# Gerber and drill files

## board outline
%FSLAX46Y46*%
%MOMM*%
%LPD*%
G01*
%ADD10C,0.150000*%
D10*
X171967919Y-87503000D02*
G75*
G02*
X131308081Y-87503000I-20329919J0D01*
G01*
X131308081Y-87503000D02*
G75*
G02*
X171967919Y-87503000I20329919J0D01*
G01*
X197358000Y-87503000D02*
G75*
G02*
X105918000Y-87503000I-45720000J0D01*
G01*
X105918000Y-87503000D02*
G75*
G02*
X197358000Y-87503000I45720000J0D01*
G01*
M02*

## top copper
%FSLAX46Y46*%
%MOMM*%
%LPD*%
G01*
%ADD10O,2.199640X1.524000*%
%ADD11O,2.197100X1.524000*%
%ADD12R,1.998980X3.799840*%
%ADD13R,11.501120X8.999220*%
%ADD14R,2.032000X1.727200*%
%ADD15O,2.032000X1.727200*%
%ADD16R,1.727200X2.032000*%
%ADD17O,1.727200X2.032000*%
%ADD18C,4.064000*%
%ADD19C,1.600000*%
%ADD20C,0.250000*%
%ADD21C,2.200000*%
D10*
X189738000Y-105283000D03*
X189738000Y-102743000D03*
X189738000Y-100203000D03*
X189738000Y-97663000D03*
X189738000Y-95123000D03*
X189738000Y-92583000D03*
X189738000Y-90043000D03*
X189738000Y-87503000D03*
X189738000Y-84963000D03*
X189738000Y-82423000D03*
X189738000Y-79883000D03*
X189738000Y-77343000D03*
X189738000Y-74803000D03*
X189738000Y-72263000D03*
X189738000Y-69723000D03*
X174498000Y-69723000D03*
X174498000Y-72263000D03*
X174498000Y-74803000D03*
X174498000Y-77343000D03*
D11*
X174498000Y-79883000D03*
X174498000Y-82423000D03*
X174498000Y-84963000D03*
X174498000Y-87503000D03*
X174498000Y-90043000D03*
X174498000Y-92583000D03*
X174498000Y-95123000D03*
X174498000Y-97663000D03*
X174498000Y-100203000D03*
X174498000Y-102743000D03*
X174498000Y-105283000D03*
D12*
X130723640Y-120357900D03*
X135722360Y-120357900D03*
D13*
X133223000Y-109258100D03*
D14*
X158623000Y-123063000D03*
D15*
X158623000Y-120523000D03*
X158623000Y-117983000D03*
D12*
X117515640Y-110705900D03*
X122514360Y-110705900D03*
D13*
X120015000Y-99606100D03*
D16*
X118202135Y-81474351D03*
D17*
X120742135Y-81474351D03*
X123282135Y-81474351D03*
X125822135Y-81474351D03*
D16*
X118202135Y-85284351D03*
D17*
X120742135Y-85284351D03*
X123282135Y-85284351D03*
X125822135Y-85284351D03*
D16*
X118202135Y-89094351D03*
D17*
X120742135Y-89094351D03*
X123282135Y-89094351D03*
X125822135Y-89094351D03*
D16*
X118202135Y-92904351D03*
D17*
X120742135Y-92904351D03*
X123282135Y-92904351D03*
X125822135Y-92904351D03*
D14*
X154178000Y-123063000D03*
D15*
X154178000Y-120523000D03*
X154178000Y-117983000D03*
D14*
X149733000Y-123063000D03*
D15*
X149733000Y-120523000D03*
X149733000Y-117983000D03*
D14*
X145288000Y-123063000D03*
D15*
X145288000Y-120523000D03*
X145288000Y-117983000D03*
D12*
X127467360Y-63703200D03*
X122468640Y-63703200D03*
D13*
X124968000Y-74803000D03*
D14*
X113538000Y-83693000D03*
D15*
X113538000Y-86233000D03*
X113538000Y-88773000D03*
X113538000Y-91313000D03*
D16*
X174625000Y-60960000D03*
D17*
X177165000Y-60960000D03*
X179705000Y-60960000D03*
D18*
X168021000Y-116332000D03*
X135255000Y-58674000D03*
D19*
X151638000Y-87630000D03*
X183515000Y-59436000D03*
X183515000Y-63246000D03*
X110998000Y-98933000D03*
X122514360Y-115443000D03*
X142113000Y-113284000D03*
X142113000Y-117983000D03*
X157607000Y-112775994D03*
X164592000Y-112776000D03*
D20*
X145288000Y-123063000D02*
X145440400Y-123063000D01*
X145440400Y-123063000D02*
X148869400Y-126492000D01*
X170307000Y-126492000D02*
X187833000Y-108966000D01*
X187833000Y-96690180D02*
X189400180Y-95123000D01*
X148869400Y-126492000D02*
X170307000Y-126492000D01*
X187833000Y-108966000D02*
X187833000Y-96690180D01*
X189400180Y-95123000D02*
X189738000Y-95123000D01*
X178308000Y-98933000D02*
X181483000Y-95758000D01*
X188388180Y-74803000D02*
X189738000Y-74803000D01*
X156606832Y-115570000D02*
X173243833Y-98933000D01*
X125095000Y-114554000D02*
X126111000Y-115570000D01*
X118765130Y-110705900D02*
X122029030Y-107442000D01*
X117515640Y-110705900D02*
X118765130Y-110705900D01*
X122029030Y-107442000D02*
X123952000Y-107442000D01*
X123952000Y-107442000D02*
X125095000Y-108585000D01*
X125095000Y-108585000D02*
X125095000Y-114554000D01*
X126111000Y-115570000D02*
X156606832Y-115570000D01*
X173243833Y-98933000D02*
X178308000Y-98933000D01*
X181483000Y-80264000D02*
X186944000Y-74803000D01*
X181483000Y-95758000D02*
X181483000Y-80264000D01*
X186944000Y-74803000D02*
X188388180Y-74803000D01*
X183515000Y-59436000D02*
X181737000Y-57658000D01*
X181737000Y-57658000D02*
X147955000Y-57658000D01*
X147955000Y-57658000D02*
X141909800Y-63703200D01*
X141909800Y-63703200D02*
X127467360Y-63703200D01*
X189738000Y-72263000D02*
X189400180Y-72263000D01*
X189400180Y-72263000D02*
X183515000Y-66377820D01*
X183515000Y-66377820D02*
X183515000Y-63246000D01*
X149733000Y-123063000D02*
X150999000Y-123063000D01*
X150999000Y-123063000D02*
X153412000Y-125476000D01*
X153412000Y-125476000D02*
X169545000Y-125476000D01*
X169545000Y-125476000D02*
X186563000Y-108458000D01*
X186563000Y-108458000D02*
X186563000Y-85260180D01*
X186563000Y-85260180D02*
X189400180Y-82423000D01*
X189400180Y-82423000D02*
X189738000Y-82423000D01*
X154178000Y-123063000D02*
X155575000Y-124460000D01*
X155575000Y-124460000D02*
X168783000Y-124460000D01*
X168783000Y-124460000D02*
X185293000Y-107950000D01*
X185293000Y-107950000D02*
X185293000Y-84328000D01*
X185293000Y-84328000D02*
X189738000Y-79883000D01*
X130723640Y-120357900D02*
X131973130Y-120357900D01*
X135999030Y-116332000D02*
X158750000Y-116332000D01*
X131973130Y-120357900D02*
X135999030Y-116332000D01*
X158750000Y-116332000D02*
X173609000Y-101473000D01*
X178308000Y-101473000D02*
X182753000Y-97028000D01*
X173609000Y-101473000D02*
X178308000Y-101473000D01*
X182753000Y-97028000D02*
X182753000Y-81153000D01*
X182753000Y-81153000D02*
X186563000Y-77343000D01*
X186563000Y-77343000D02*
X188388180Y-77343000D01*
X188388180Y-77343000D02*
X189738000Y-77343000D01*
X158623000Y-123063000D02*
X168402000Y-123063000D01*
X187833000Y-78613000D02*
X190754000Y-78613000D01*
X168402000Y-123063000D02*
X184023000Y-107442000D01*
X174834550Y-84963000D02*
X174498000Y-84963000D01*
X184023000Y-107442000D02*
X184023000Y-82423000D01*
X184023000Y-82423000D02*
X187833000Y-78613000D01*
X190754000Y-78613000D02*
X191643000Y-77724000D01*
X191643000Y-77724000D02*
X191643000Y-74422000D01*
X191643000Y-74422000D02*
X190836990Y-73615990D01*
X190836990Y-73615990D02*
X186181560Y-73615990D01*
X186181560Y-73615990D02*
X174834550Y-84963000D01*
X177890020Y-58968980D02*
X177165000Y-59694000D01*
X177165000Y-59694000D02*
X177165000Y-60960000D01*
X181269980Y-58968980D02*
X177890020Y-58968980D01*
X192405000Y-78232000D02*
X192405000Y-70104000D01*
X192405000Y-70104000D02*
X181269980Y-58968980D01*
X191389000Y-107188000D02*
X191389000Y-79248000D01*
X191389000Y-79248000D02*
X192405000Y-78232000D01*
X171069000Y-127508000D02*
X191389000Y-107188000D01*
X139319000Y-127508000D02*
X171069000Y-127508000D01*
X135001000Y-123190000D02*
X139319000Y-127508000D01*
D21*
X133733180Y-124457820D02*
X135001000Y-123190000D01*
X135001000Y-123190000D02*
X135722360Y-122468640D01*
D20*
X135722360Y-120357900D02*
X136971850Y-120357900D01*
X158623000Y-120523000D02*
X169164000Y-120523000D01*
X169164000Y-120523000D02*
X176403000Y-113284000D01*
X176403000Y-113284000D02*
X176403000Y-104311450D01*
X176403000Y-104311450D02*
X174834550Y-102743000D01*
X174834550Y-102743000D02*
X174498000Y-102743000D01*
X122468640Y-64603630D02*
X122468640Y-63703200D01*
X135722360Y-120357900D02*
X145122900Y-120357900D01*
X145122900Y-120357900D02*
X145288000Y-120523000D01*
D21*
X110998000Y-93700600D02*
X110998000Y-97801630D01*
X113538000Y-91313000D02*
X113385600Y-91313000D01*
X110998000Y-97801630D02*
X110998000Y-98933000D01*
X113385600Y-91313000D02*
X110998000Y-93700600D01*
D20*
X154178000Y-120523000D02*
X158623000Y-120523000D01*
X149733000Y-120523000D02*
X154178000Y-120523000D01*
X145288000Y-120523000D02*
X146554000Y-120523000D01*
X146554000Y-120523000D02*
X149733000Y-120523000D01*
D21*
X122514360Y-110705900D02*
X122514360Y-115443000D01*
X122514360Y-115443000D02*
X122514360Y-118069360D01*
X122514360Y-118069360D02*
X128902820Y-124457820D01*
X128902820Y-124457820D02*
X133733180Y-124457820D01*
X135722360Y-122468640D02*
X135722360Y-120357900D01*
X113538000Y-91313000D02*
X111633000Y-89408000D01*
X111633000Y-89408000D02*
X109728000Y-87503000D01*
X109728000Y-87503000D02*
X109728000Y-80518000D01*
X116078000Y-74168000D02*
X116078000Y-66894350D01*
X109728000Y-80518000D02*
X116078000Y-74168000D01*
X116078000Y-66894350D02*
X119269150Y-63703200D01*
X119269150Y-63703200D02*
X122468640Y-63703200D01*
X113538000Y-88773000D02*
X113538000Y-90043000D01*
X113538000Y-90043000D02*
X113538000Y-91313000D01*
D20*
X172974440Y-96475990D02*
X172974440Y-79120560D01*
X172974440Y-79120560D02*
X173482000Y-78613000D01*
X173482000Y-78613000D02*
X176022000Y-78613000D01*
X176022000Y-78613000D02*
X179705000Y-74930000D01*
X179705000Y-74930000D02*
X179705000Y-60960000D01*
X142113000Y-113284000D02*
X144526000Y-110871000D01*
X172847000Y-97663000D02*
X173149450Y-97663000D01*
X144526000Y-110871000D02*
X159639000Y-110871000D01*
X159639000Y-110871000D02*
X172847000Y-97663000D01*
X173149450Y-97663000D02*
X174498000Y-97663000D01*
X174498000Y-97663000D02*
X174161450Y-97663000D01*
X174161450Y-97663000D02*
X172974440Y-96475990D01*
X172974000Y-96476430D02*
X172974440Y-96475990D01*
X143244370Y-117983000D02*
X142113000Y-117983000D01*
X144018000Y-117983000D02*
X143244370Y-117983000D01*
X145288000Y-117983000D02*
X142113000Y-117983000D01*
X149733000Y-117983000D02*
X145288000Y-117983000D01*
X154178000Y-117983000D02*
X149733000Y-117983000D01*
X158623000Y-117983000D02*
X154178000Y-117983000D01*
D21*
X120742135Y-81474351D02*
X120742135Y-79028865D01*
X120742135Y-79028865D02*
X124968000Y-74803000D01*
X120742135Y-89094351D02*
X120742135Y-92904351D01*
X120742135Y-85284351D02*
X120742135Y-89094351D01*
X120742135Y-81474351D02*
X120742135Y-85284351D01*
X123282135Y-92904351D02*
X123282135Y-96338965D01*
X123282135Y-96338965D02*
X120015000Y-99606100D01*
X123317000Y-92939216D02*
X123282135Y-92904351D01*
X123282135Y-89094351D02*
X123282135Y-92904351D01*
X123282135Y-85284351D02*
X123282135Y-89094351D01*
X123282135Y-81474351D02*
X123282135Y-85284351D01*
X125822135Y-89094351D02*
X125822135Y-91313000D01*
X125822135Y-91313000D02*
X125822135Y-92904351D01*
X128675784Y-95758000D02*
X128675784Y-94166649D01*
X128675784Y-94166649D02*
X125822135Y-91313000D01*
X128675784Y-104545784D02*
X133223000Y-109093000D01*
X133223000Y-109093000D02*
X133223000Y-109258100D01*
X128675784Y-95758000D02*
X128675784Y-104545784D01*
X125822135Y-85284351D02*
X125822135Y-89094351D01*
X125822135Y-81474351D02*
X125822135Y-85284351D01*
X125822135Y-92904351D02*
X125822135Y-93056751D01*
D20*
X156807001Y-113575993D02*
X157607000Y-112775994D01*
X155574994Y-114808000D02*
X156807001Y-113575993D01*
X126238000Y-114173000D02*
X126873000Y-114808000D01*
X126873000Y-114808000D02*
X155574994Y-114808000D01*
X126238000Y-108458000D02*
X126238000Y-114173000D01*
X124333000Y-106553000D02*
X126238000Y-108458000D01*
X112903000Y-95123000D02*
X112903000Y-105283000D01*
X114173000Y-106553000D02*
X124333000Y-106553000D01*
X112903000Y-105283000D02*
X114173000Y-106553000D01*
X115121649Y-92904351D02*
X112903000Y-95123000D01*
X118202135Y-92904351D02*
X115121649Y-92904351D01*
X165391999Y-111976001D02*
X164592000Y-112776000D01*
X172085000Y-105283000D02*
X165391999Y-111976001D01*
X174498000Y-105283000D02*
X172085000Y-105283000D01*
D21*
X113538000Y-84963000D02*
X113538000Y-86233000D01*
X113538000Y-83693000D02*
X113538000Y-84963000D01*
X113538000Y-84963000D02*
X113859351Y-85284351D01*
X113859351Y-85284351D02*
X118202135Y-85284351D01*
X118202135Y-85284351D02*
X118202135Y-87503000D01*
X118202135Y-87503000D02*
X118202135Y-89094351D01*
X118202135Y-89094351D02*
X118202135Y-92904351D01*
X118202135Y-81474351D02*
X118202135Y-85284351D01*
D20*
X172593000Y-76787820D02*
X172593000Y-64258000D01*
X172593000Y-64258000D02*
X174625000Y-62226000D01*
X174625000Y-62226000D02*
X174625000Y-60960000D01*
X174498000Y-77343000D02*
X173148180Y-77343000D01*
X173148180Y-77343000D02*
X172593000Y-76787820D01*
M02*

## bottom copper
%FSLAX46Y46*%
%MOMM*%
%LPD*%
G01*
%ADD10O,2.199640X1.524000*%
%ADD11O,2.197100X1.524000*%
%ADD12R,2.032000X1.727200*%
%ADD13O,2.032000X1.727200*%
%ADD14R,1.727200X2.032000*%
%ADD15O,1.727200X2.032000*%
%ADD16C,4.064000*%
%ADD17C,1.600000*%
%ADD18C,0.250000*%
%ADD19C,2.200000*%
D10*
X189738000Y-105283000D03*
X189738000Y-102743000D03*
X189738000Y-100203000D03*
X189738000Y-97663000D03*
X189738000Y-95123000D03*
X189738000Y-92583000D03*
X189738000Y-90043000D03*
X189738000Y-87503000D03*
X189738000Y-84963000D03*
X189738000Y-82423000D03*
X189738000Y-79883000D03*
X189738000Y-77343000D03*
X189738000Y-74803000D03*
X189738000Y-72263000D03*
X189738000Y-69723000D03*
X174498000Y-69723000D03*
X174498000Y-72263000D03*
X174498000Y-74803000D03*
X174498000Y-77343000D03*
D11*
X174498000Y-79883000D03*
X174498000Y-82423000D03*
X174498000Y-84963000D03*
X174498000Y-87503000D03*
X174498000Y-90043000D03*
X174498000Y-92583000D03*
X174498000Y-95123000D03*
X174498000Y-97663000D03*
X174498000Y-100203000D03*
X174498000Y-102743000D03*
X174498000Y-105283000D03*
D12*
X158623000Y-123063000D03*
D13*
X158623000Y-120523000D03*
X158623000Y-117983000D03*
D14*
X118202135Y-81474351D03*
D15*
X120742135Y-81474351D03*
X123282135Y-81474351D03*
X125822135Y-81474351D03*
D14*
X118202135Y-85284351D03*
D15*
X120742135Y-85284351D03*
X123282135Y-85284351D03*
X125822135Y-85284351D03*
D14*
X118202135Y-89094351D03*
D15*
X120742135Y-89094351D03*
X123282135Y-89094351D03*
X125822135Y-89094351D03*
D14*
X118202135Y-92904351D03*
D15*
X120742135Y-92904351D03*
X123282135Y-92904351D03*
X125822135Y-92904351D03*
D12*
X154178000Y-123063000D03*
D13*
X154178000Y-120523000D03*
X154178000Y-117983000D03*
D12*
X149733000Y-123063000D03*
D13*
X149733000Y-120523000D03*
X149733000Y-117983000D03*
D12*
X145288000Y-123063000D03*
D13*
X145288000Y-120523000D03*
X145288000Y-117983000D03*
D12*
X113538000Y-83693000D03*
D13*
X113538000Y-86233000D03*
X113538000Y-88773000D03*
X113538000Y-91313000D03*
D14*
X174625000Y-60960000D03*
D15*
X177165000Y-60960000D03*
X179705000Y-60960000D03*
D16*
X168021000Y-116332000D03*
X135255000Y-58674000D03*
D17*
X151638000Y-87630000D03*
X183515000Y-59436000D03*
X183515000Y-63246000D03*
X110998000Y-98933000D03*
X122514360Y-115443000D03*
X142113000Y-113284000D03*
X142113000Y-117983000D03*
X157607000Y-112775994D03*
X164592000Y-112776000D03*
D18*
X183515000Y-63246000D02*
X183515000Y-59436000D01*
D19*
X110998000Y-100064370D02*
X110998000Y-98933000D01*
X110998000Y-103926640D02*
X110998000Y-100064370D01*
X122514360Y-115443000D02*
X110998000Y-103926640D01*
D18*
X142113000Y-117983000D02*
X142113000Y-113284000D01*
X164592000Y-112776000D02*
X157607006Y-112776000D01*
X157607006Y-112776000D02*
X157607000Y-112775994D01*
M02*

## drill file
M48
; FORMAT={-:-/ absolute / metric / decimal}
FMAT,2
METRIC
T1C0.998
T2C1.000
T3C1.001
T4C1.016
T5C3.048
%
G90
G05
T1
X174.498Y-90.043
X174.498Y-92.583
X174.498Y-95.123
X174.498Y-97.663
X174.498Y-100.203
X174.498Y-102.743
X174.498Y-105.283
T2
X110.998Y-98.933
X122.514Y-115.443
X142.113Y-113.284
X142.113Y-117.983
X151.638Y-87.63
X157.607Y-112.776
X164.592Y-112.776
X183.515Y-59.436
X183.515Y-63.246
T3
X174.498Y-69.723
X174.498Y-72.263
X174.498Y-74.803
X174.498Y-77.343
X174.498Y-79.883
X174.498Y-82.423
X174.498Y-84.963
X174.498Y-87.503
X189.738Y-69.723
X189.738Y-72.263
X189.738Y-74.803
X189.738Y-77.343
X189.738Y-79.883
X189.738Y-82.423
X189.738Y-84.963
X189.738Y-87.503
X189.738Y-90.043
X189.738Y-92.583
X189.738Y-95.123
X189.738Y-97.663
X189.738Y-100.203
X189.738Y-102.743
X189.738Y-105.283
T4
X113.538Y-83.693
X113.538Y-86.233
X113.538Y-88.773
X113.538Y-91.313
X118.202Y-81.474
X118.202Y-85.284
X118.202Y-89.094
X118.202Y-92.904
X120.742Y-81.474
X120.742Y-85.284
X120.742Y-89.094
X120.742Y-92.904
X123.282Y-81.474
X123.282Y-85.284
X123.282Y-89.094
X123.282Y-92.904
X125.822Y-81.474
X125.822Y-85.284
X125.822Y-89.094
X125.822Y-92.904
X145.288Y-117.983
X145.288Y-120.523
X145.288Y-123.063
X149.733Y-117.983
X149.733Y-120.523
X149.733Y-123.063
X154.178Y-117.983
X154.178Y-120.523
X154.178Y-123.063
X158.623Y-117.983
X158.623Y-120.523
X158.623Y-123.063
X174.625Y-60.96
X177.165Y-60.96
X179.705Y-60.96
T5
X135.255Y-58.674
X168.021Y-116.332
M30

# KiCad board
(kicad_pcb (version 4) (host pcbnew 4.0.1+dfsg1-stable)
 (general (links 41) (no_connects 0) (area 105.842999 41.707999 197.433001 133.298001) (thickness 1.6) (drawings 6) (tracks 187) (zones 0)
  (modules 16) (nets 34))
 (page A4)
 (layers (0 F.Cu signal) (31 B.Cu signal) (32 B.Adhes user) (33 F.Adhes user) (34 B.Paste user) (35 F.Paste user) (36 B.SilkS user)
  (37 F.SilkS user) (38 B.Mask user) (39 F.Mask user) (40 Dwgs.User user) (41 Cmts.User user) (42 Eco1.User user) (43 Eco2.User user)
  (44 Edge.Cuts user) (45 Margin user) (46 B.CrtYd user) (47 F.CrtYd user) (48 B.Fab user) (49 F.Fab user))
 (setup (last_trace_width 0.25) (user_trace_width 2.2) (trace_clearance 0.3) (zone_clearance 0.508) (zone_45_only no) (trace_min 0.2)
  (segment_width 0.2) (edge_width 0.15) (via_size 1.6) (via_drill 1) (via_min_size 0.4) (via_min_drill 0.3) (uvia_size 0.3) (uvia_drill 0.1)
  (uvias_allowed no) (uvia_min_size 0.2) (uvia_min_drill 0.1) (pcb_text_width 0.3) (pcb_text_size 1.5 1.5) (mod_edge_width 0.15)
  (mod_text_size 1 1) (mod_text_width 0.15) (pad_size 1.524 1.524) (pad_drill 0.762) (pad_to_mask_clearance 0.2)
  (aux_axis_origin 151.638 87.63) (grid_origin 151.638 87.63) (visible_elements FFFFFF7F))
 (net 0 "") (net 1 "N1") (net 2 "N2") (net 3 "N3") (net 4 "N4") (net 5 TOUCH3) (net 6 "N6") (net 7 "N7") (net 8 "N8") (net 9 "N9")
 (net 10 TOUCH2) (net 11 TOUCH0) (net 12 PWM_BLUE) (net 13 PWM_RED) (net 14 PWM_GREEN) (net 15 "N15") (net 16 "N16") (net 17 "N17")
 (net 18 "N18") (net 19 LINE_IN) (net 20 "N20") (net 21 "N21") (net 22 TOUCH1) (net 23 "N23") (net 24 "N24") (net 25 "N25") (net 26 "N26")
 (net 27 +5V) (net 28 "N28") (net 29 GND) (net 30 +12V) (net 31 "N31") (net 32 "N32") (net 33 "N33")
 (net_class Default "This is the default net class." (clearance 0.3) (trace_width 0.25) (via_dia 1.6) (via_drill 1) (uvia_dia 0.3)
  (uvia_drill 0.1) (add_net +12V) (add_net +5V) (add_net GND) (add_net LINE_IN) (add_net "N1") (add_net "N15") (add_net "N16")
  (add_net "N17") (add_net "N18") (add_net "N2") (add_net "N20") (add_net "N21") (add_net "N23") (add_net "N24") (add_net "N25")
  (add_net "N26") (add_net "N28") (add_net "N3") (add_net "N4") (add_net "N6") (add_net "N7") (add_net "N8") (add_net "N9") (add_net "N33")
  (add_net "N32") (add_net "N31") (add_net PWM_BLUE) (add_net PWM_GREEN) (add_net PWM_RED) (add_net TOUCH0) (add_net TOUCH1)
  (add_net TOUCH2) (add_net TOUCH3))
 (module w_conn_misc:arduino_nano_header (layer F.Cu) (at 182.118 87.503 90)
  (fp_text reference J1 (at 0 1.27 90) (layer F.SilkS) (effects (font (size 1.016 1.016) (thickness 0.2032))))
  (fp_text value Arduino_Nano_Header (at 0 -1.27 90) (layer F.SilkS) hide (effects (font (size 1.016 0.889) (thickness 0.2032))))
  (pad 1 thru_hole oval (at -17.78 7.62 90) (size 1.524 2.19964) (drill 1.00076) (layers *.Cu *.Mask F.SilkS) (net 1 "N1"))
  (pad 2 thru_hole oval (at -15.24 7.62 90) (size 1.524 2.19964) (drill 1.00076) (layers *.Cu *.Mask F.SilkS) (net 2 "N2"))
  (pad 3 thru_hole oval (at -12.7 7.62 90) (size 1.524 2.19964) (drill 1.00076) (layers *.Cu *.Mask F.SilkS) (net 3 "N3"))
  (pad 4 thru_hole oval (at -10.16 7.62 90) (size 1.524 2.19964) (drill 1.00076) (layers *.Cu *.Mask F.SilkS) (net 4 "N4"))
  (pad 5 thru_hole oval (at -7.62 7.62 90) (size 1.524 2.19964) (drill 1.00076) (layers *.Cu *.Mask F.SilkS) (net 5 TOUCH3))
  (pad 6 thru_hole oval (at -5.08 7.62 90) (size 1.524 2.19964) (drill 1.00076) (layers *.Cu *.Mask F.SilkS) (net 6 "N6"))
  (pad 7 thru_hole oval (at -2.54 7.62 90) (size 1.524 2.19964) (drill 1.00076) (layers *.Cu *.Mask F.SilkS) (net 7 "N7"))
  (pad 8 thru_hole oval (at 0 7.62 90) (size 1.524 2.19964) (drill 1.00076) (layers *.Cu *.Mask F.SilkS) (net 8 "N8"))
  (pad 9 thru_hole oval (at 2.54 7.62 90) (size 1.524 2.19964) (drill 1.00076) (layers *.Cu *.Mask F.SilkS) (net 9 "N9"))
  (pad 10 thru_hole oval (at 5.08 7.62 90) (size 1.524 2.19964) (drill 1.00076) (layers *.Cu *.Mask F.SilkS) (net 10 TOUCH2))
  (pad 11 thru_hole oval (at 7.62 7.62 90) (size 1.524 2.19964) (drill 1.00076) (layers *.Cu *.Mask F.SilkS) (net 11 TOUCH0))
  (pad 12 thru_hole oval (at 10.16 7.62 90) (size 1.524 2.19964) (drill 1.00076) (layers *.Cu *.Mask F.SilkS) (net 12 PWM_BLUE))
  (pad 13 thru_hole oval (at 12.7 7.62 90) (size 1.524 2.19964) (drill 1.00076) (layers *.Cu *.Mask F.SilkS) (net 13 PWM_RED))
  (pad 14 thru_hole oval (at 15.24 7.62 90) (size 1.524 2.19964) (drill 1.00076) (layers *.Cu *.Mask F.SilkS) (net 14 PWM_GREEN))
  (pad 15 thru_hole oval (at 17.78 7.62 90) (size 1.524 2.19964) (drill 1.00076) (layers *.Cu *.Mask F.SilkS) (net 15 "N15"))
  (pad 16 thru_hole oval (at 17.78 -7.62 90) (size 1.524 2.19964) (drill 1.00076) (layers *.Cu *.Mask F.SilkS) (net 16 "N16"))
  (pad 17 thru_hole oval (at 15.24 -7.62 90) (size 1.524 2.19964) (drill 1.00076) (layers *.Cu *.Mask F.SilkS) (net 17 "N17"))
  (pad 18 thru_hole oval (at 12.7 -7.62 90) (size 1.524 2.19964) (drill 1.00076) (layers *.Cu *.Mask F.SilkS) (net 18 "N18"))
  (pad 19 thru_hole oval (at 10.16 -7.62 90) (size 1.524 2.19964) (drill 1.00076) (layers *.Cu *.Mask F.SilkS) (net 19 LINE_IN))
  (pad 20 thru_hole oval (at 7.62 -7.62 90) (size 1.524 2.1971) (drill 1.00076) (layers *.Cu *.Mask F.SilkS) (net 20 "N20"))
  (pad 21 thru_hole oval (at 5.08 -7.62 90) (size 1.524 2.1971) (drill 1.00076) (layers *.Cu *.Mask F.SilkS) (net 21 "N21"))
  (pad 22 thru_hole oval (at 2.54 -7.62 90) (size 1.524 2.1971) (drill 1.00076) (layers *.Cu *.Mask F.SilkS) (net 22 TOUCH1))
  (pad 23 thru_hole oval (at 0 -7.62 90) (size 1.524 2.1971) (drill 1.00076) (layers *.Cu *.Mask F.SilkS) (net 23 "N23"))
  (pad 24 thru_hole oval (at -2.54 -7.62 90) (size 1.524 2.1971) (drill 0.99822) (layers *.Cu *.Mask F.SilkS) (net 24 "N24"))
  (pad 25 thru_hole oval (at -5.08 -7.62 90) (size 1.524 2.1971) (drill 0.99822) (layers *.Cu *.Mask F.SilkS) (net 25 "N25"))
  (pad 26 thru_hole oval (at -7.62 -7.62 90) (size 1.524 2.1971) (drill 0.99822) (layers *.Cu *.Mask F.SilkS) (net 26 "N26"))
  (pad 27 thru_hole oval (at -10.16 -7.62 90) (size 1.524 2.1971) (drill 0.99822) (layers *.Cu *.Mask F.SilkS) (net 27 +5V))
  (pad 28 thru_hole oval (at -12.7 -7.62 90) (size 1.524 2.1971) (drill 0.99822) (layers *.Cu *.Mask F.SilkS) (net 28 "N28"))
  (pad 29 thru_hole oval (at -15.24 -7.62 90) (size 1.524 2.1971) (drill 0.99822) (layers *.Cu *.Mask F.SilkS) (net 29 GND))
  (pad 30 thru_hole oval (at -17.78 -7.62 90) (size 1.524 2.1971) (drill 0.99822) (layers *.Cu *.Mask F.SilkS) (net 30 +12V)))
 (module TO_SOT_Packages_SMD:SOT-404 (layer F.Cu) (at 133.223 114.808)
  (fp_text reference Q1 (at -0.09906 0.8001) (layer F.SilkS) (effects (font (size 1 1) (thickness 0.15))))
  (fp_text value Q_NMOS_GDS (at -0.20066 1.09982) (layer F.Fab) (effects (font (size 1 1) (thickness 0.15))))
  (pad 1 smd rect (at -2.49936 5.5499) (size 1.99898 3.79984) (layers F.Cu F.Paste F.Mask) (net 12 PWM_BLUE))
  (pad 3 smd rect (at 2.49936 5.5499) (size 1.99898 3.79984) (layers F.Cu F.Paste F.Mask) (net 29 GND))
  (pad 2 smd rect (at 0 -5.5499) (size 11.50112 8.99922) (layers F.Cu F.Paste F.Mask) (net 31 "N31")))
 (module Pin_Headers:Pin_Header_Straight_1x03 (layer F.Cu) (at 158.623 123.063 180)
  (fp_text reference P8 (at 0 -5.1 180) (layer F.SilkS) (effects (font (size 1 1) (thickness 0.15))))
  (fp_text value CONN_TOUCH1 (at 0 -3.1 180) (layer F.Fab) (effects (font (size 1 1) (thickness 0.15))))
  (pad 1 thru_hole rect (at 0 0 180) (size 2.032 1.7272) (drill 1.016) (layers *.Cu *.Mask F.SilkS) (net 22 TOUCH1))
  (pad 2 thru_hole oval (at 0 2.54 180) (size 2.032 1.7272) (drill 1.016) (layers *.Cu *.Mask F.SilkS) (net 29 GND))
  (pad 3 thru_hole oval (at 0 5.08 180) (size 2.032 1.7272) (drill 1.016) (layers *.Cu *.Mask F.SilkS) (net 27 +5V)))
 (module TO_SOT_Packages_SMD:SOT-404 (layer F.Cu) (at 120.015 105.156)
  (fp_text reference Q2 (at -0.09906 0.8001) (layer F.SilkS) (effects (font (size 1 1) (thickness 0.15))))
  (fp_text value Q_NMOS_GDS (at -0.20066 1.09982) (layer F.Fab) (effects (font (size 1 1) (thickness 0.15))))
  (pad 1 smd rect (at -2.49936 5.5499) (size 1.99898 3.79984) (layers F.Cu F.Paste F.Mask) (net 13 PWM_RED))
  (pad 3 smd rect (at 2.49936 5.5499) (size 1.99898 3.79984) (layers F.Cu F.Paste F.Mask) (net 29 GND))
  (pad 2 smd rect (at 0 -5.5499) (size 11.50112 8.99922) (layers F.Cu F.Paste F.Mask) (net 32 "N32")))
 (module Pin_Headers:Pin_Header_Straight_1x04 (layer F.Cu) (at 118.202135 81.474351 90)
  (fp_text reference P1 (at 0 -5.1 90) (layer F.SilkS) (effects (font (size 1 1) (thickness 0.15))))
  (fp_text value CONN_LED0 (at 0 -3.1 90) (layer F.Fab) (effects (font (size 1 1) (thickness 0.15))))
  (pad 1 thru_hole rect (at 0 0 90) (size 2.032 1.7272) (drill 1.016) (layers *.Cu *.Mask F.SilkS) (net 30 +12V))
  (pad 2 thru_hole oval (at 0 2.54 90) (size 2.032 1.7272) (drill 1.016) (layers *.Cu *.Mask F.SilkS) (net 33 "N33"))
  (pad 3 thru_hole oval (at 0 5.08 90) (size 2.032 1.7272) (drill 1.016) (layers *.Cu *.Mask F.SilkS) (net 32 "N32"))
  (pad 4 thru_hole oval (at 0 7.62 90) (size 2.032 1.7272) (drill 1.016) (layers *.Cu *.Mask F.SilkS) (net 31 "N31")))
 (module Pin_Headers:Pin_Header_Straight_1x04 (layer F.Cu) (at 118.202135 85.284351 90)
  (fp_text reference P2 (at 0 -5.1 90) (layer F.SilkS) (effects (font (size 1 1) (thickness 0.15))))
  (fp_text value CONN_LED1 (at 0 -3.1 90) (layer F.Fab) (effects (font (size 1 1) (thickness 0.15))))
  (pad 1 thru_hole rect (at 0 0 90) (size 2.032 1.7272) (drill 1.016) (layers *.Cu *.Mask F.SilkS) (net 30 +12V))
  (pad 2 thru_hole oval (at 0 2.54 90) (size 2.032 1.7272) (drill 1.016) (layers *.Cu *.Mask F.SilkS) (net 33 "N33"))
  (pad 3 thru_hole oval (at 0 5.08 90) (size 2.032 1.7272) (drill 1.016) (layers *.Cu *.Mask F.SilkS) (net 32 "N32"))
  (pad 4 thru_hole oval (at 0 7.62 90) (size 2.032 1.7272) (drill 1.016) (layers *.Cu *.Mask F.SilkS) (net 31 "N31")))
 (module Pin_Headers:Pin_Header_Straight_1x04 (layer F.Cu) (at 118.202135 89.094351 90)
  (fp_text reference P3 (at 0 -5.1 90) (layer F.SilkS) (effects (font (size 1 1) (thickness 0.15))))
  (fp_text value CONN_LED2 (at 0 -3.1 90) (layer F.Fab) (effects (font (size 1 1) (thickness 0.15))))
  (pad 1 thru_hole rect (at 0 0 90) (size 2.032 1.7272) (drill 1.016) (layers *.Cu *.Mask F.SilkS) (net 30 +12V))
  (pad 2 thru_hole oval (at 0 2.54 90) (size 2.032 1.7272) (drill 1.016) (layers *.Cu *.Mask F.SilkS) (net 33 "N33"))
  (pad 3 thru_hole oval (at 0 5.08 90) (size 2.032 1.7272) (drill 1.016) (layers *.Cu *.Mask F.SilkS) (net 32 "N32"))
  (pad 4 thru_hole oval (at 0 7.62 90) (size 2.032 1.7272) (drill 1.016) (layers *.Cu *.Mask F.SilkS) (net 31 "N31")))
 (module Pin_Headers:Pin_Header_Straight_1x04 (layer F.Cu) (at 118.202135 92.904351 90)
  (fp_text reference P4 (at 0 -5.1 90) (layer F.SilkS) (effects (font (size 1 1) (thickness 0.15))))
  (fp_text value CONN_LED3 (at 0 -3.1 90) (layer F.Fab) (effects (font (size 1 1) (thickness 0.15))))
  (pad 1 thru_hole rect (at 0 0 90) (size 2.032 1.7272) (drill 1.016) (layers *.Cu *.Mask F.SilkS) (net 30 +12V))
  (pad 2 thru_hole oval (at 0 2.54 90) (size 2.032 1.7272) (drill 1.016) (layers *.Cu *.Mask F.SilkS) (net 33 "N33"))
  (pad 3 thru_hole oval (at 0 5.08 90) (size 2.032 1.7272) (drill 1.016) (layers *.Cu *.Mask F.SilkS) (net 32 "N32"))
  (pad 4 thru_hole oval (at 0 7.62 90) (size 2.032 1.7272) (drill 1.016) (layers *.Cu *.Mask F.SilkS) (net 31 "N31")))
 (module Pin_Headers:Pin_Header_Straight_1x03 (layer F.Cu) (at 154.178 123.063 180)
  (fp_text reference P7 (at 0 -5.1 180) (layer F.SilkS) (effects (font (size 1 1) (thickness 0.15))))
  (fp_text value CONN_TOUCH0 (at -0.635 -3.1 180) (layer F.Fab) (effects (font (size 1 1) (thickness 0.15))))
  (pad 1 thru_hole rect (at 0 0 180) (size 2.032 1.7272) (drill 1.016) (layers *.Cu *.Mask F.SilkS) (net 11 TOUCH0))
  (pad 2 thru_hole oval (at 0 2.54 180) (size 2.032 1.7272) (drill 1.016) (layers *.Cu *.Mask F.SilkS) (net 29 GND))
  (pad 3 thru_hole oval (at 0 5.08 180) (size 2.032 1.7272) (drill 1.016) (layers *.Cu *.Mask F.SilkS) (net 27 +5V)))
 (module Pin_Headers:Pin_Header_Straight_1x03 (layer F.Cu) (at 149.733 123.063 180)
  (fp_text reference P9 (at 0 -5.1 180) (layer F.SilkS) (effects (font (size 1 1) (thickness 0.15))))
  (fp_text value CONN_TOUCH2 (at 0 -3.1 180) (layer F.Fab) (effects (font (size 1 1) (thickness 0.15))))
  (pad 1 thru_hole rect (at 0 0 180) (size 2.032 1.7272) (drill 1.016) (layers *.Cu *.Mask F.SilkS) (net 10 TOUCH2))
  (pad 2 thru_hole oval (at 0 2.54 180) (size 2.032 1.7272) (drill 1.016) (layers *.Cu *.Mask F.SilkS) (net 29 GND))
  (pad 3 thru_hole oval (at 0 5.08 180) (size 2.032 1.7272) (drill 1.016) (layers *.Cu *.Mask F.SilkS) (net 27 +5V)))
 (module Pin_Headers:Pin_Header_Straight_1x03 (layer F.Cu) (at 145.288 123.063 180)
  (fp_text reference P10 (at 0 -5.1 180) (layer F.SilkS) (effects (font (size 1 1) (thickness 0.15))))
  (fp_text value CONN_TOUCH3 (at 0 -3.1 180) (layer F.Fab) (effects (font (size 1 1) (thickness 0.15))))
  (pad 1 thru_hole rect (at 0 0 180) (size 2.032 1.7272) (drill 1.016) (layers *.Cu *.Mask F.SilkS) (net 5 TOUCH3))
  (pad 2 thru_hole oval (at 0 2.54 180) (size 2.032 1.7272) (drill 1.016) (layers *.Cu *.Mask F.SilkS) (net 29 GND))
  (pad 3 thru_hole oval (at 0 5.08 180) (size 2.032 1.7272) (drill 1.016) (layers *.Cu *.Mask F.SilkS) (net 27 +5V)))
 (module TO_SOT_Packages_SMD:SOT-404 (layer F.Cu) (at 124.968 69.2531 180)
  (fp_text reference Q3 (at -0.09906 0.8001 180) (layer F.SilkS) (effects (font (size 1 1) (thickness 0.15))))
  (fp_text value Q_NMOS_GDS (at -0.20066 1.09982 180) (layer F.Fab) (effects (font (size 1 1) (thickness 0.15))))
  (pad 1 smd rect (at -2.49936 5.5499 180) (size 1.99898 3.79984) (layers F.Cu F.Paste F.Mask) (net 14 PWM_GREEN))
  (pad 3 smd rect (at 2.49936 5.5499 180) (size 1.99898 3.79984) (layers F.Cu F.Paste F.Mask) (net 29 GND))
  (pad 2 smd rect (at 0 -5.5499 180) (size 11.50112 8.99922) (layers F.Cu F.Paste F.Mask) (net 33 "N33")))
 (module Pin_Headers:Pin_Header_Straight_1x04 (layer F.Cu) (at 113.538 83.693)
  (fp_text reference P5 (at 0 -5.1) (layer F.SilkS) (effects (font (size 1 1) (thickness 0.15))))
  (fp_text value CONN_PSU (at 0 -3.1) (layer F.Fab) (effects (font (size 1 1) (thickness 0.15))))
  (pad 1 thru_hole rect (at 0 0) (size 2.032 1.7272) (drill 1.016) (layers *.Cu *.Mask F.SilkS) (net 30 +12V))
  (pad 2 thru_hole oval (at 0 2.54) (size 2.032 1.7272) (drill 1.016) (layers *.Cu *.Mask F.SilkS) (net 30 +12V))
  (pad 3 thru_hole oval (at 0 5.08) (size 2.032 1.7272) (drill 1.016) (layers *.Cu *.Mask F.SilkS) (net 29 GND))
  (pad 4 thru_hole oval (at 0 7.62) (size 2.032 1.7272) (drill 1.016) (layers *.Cu *.Mask F.SilkS) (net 29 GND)))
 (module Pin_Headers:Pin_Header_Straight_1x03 (layer F.Cu) (at 174.625 60.96 90)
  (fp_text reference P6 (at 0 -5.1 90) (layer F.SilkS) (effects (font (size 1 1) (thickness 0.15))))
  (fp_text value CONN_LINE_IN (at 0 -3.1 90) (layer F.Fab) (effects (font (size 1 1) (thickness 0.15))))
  (pad 1 thru_hole rect (at 0 0 90) (size 2.032 1.7272) (drill 1.016) (layers *.Cu *.Mask F.SilkS) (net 19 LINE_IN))
  (pad 2 thru_hole oval (at 0 2.54 90) (size 2.032 1.7272) (drill 1.016) (layers *.Cu *.Mask F.SilkS) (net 29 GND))
  (pad 3 thru_hole oval (at 0 5.08 90) (size 2.032 1.7272) (drill 1.016) (layers *.Cu *.Mask F.SilkS) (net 27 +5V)))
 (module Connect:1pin (layer F.Cu) (at 168.021 116.332)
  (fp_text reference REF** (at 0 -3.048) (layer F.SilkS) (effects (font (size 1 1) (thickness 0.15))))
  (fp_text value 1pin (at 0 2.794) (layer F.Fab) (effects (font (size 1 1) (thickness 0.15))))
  (pad 1 thru_hole circle (at 0 0) (size 4.064 4.064) (drill 3.048) (layers *.Cu *.Mask F.SilkS)))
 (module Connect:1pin (layer F.Cu) (at 135.255 58.674)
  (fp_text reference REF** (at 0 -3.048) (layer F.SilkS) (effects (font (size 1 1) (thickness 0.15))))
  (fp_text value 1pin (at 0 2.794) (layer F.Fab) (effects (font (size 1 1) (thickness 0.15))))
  (pad 1 thru_hole circle (at 0 0) (size 4.064 4.064) (drill 3.048) (layers *.Cu *.Mask F.SilkS)))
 (gr_circle (center 151.638 87.503) (end 171.958 88.138) (layer Edge.Cuts) (width 0.15))
 (gr_circle (center 151.638 87.503) (end 197.358 87.503) (layer Edge.Cuts) (width 0.15))
 (via (at 151.638 87.63) (size 1.6) (drill 1) (layers F.Cu B.Cu) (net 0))
 (segment (start 145.288 123.063) (end 145.4404 123.063) (width 0.25) (layer F.Cu) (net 5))
 (segment (start 145.4404 123.063) (end 148.8694 126.492) (width 0.25) (layer F.Cu) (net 5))
 (segment (start 170.307 126.492) (end 187.833 108.966) (width 0.25) (layer F.Cu) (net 5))
 (segment (start 187.833 96.69018) (end 189.40018 95.123) (width 0.25) (layer F.Cu) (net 5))
 (segment (start 148.8694 126.492) (end 170.307 126.492) (width 0.25) (layer F.Cu) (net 5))
 (segment (start 187.833 108.966) (end 187.833 96.69018) (width 0.25) (layer F.Cu) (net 5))
 (segment (start 189.40018 95.123) (end 189.738 95.123) (width 0.25) (layer F.Cu) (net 5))
 (segment (start 178.308 98.933) (end 181.483 95.758) (width 0.25) (layer F.Cu) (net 13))
 (segment (start 188.38818 74.803) (end 189.738 74.803) (width 0.25) (layer F.Cu) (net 13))
 (segment (start 156.606832 115.57) (end 173.243833 98.933) (width 0.25) (layer F.Cu) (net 13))
 (segment (start 125.095 114.554) (end 126.111 115.57) (width 0.25) (layer F.Cu) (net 13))
 (segment (start 118.76513 110.7059) (end 122.02903 107.442) (width 0.25) (layer F.Cu) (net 13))
 (segment (start 117.51564 110.7059) (end 118.76513 110.7059) (width 0.25) (layer F.Cu) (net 13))
 (segment (start 122.02903 107.442) (end 123.952 107.442) (width 0.25) (layer F.Cu) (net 13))
 (segment (start 123.952 107.442) (end 125.095 108.585) (width 0.25) (layer F.Cu) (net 13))
 (segment (start 125.095 108.585) (end 125.095 114.554) (width 0.25) (layer F.Cu) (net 13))
 (segment (start 126.111 115.57) (end 156.606832 115.57) (width 0.25) (layer F.Cu) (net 13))
 (segment (start 173.243833 98.933) (end 178.308 98.933) (width 0.25) (layer F.Cu) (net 13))
 (segment (start 181.483 80.264) (end 186.944 74.803) (width 0.25) (layer F.Cu) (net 13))
 (segment (start 181.483 95.758) (end 181.483 80.264) (width 0.25) (layer F.Cu) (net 13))
 (segment (start 186.944 74.803) (end 188.38818 74.803) (width 0.25) (layer F.Cu) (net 13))
 (segment (start 183.515 59.436) (end 181.737 57.658) (width 0.25) (layer F.Cu) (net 14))
 (segment (start 181.737 57.658) (end 147.955 57.658) (width 0.25) (layer F.Cu) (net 14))
 (segment (start 147.955 57.658) (end 141.9098 63.7032) (width 0.25) (layer F.Cu) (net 14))
 (segment (start 141.9098 63.7032) (end 127.46736 63.7032) (width 0.25) (layer F.Cu) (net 14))
 (segment (start 183.515 63.246) (end 183.515 59.436) (width 0.25) (layer B.Cu) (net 14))
 (via (at 183.515 59.436) (size 1.6) (drill 1) (layers F.Cu B.Cu) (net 14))
 (segment (start 189.738 72.263) (end 189.40018 72.263) (width 0.25) (layer F.Cu) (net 14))
 (via (at 183.515 63.246) (size 1.6) (drill 1) (layers F.Cu B.Cu) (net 14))
 (segment (start 189.40018 72.263) (end 183.515 66.37782) (width 0.25) (layer F.Cu) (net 14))
 (segment (start 183.515 66.37782) (end 183.515 63.246) (width 0.25) (layer F.Cu) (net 14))
 (segment (start 149.733 123.063) (end 150.999 123.063) (width 0.25) (layer F.Cu) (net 10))
 (segment (start 150.999 123.063) (end 153.412 125.476) (width 0.25) (layer F.Cu) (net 10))
 (segment (start 153.412 125.476) (end 169.545 125.476) (width 0.25) (layer F.Cu) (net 10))
 (segment (start 169.545 125.476) (end 186.563 108.458) (width 0.25) (layer F.Cu) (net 10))
 (segment (start 186.563 108.458) (end 186.563 85.26018) (width 0.25) (layer F.Cu) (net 10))
 (segment (start 186.563 85.26018) (end 189.40018 82.423) (width 0.25) (layer F.Cu) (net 10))
 (segment (start 189.40018 82.423) (end 189.738 82.423) (width 0.25) (layer F.Cu) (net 10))
 (segment (start 154.178 123.063) (end 155.575 124.46) (width 0.25) (layer F.Cu) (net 11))
 (segment (start 155.575 124.46) (end 168.783 124.46) (width 0.25) (layer F.Cu) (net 11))
 (segment (start 168.783 124.46) (end 185.293 107.95) (width 0.25) (layer F.Cu) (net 11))
 (segment (start 185.293 107.95) (end 185.293 84.328) (width 0.25) (layer F.Cu) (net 11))
 (segment (start 185.293 84.328) (end 189.738 79.883) (width 0.25) (layer F.Cu) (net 11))
 (segment (start 130.72364 120.3579) (end 131.97313 120.3579) (width 0.25) (layer F.Cu) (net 12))
 (segment (start 135.99903 116.332) (end 158.75 116.332) (width 0.25) (layer F.Cu) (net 12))
 (segment (start 131.97313 120.3579) (end 135.99903 116.332) (width 0.25) (layer F.Cu) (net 12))
 (segment (start 158.75 116.332) (end 173.609 101.473) (width 0.25) (layer F.Cu) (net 12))
 (segment (start 178.308 101.473) (end 182.753 97.028) (width 0.25) (layer F.Cu) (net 12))
 (segment (start 173.609 101.473) (end 178.308 101.473) (width 0.25) (layer F.Cu) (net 12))
 (segment (start 182.753 97.028) (end 182.753 81.153) (width 0.25) (layer F.Cu) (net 12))
 (segment (start 182.753 81.153) (end 186.563 77.343) (width 0.25) (layer F.Cu) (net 12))
 (segment (start 186.563 77.343) (end 188.38818 77.343) (width 0.25) (layer F.Cu) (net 12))
 (segment (start 188.38818 77.343) (end 189.738 77.343) (width 0.25) (layer F.Cu) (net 12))
 (segment (start 158.623 123.063) (end 168.402 123.063) (width 0.25) (layer F.Cu) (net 22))
 (segment (start 187.833 78.613) (end 190.754 78.613) (width 0.25) (layer F.Cu) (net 22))
 (segment (start 168.402 123.063) (end 184.023 107.442) (width 0.25) (layer F.Cu) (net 22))
 (segment (start 174.83455 84.963) (end 174.498 84.963) (width 0.25) (layer F.Cu) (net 22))
 (segment (start 184.023 107.442) (end 184.023 82.423) (width 0.25) (layer F.Cu) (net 22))
 (segment (start 184.023 82.423) (end 187.833 78.613) (width 0.25) (layer F.Cu) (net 22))
 (segment (start 190.754 78.613) (end 191.643 77.724) (width 0.25) (layer F.Cu) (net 22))
 (segment (start 191.643 77.724) (end 191.643 74.422) (width 0.25) (layer F.Cu) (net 22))
 (segment (start 191.643 74.422) (end 190.83699 73.61599) (width 0.25) (layer F.Cu) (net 22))
 (segment (start 190.83699 73.61599) (end 186.18156 73.61599) (width 0.25) (layer F.Cu) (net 22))
 (segment (start 186.18156 73.61599) (end 174.83455 84.963) (width 0.25) (layer F.Cu) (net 22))
 (segment (start 177.89002 58.96898) (end 177.165 59.694) (width 0.25) (layer F.Cu) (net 29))
 (segment (start 177.165 59.694) (end 177.165 60.96) (width 0.25) (layer F.Cu) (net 29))
 (segment (start 181.26998 58.96898) (end 177.89002 58.96898) (width 0.25) (layer F.Cu) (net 29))
 (segment (start 192.405 78.232) (end 192.405 70.104) (width 0.25) (layer F.Cu) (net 29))
 (segment (start 192.405 70.104) (end 181.26998 58.96898) (width 0.25) (layer F.Cu) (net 29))
 (segment (start 191.389 107.188) (end 191.389 79.248) (width 0.25) (layer F.Cu) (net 29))
 (segment (start 191.389 79.248) (end 192.405 78.232) (width 0.25) (layer F.Cu) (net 29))
 (segment (start 171.069 127.508) (end 191.389 107.188) (width 0.25) (layer F.Cu) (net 29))
 (segment (start 139.319 127.508) (end 171.069 127.508) (width 0.25) (layer F.Cu) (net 29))
 (segment (start 135.001 123.19) (end 139.319 127.508) (width 0.25) (layer F.Cu) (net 29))
 (segment (start 133.73318 124.45782) (end 135.001 123.19) (width 2.2) (layer F.Cu) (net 29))
 (segment (start 135.001 123.19) (end 135.72236 122.46864) (width 2.2) (layer F.Cu) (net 29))
 (segment (start 135.72236 120.3579) (end 136.97185 120.3579) (width 0.25) (layer F.Cu) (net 29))
 (segment (start 158.623 120.523) (end 169.164 120.523) (width 0.25) (layer F.Cu) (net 29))
 (segment (start 169.164 120.523) (end 176.403 113.284) (width 0.25) (layer F.Cu) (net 29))
 (segment (start 176.403 113.284) (end 176.403 104.31145) (width 0.25) (layer F.Cu) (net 29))
 (segment (start 176.403 104.31145) (end 174.83455 102.743) (width 0.25) (layer F.Cu) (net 29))
 (segment (start 174.83455 102.743) (end 174.498 102.743) (width 0.25) (layer F.Cu) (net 29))
 (segment (start 122.46864 64.60363) (end 122.46864 63.7032) (width 0.25) (layer F.Cu) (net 29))
 (segment (start 135.72236 120.3579) (end 145.1229 120.3579) (width 0.25) (layer F.Cu) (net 29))
 (segment (start 145.1229 120.3579) (end 145.288 120.523) (width 0.25) (layer F.Cu) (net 29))
 (segment (start 110.998 100.06437) (end 110.998 98.933) (width 2.2) (layer B.Cu) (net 29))
 (segment (start 110.998 103.92664) (end 110.998 100.06437) (width 2.2) (layer B.Cu) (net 29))
 (segment (start 122.51436 115.443) (end 110.998 103.92664) (width 2.2) (layer B.Cu) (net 29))
 (segment (start 110.998 93.7006) (end 110.998 97.80163) (width 2.2) (layer F.Cu) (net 29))
 (segment (start 113.538 91.313) (end 113.3856 91.313) (width 2.2) (layer F.Cu) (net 29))
 (segment (start 110.998 97.80163) (end 110.998 98.933) (width 2.2) (layer F.Cu) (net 29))
 (segment (start 113.3856 91.313) (end 110.998 93.7006) (width 2.2) (layer F.Cu) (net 29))
 (via (at 110.998 98.933) (size 1.6) (drill 1) (layers F.Cu B.Cu) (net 29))
 (segment (start 154.178 120.523) (end 158.623 120.523) (width 0.25) (layer F.Cu) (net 29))
 (segment (start 149.733 120.523) (end 154.178 120.523) (width 0.25) (layer F.Cu) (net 29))
 (segment (start 145.288 120.523) (end 146.554 120.523) (width 0.25) (layer F.Cu) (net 29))
 (segment (start 146.554 120.523) (end 149.733 120.523) (width 0.25) (layer F.Cu) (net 29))
 (segment (start 122.51436 110.7059) (end 122.51436 115.443) (width 2.2) (layer F.Cu) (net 29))
 (segment (start 122.51436 115.443) (end 122.51436 118.06936) (width 2.2) (layer F.Cu) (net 29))
 (via (at 122.51436 115.443) (size 1.6) (drill 1) (layers F.Cu B.Cu) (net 29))
 (segment (start 122.51436 118.06936) (end 128.90282 124.45782) (width 2.2) (layer F.Cu) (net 29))
 (segment (start 128.90282 124.45782) (end 133.73318 124.45782) (width 2.2) (layer F.Cu) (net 29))
 (segment (start 135.72236 122.46864) (end 135.72236 120.3579) (width 2.2) (layer F.Cu) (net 29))
 (segment (start 113.538 91.313) (end 111.633 89.408) (width 2.2) (layer F.Cu) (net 29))
 (segment (start 111.633 89.408) (end 109.728 87.503) (width 2.2) (layer F.Cu) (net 29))
 (segment (start 109.728 87.503) (end 109.728 80.518) (width 2.2) (layer F.Cu) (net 29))
 (segment (start 116.078 74.168) (end 116.078 66.89435) (width 2.2) (layer F.Cu) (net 29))
 (segment (start 109.728 80.518) (end 116.078 74.168) (width 2.2) (layer F.Cu) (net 29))
 (segment (start 116.078 66.89435) (end 119.26915 63.7032) (width 2.2) (layer F.Cu) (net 29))
 (segment (start 119.26915 63.7032) (end 122.46864 63.7032) (width 2.2) (layer F.Cu) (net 29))
 (segment (start 113.538 88.773) (end 113.538 90.043) (width 2.2) (layer F.Cu) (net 29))
 (segment (start 113.538 90.043) (end 113.538 91.313) (width 2.2) (layer F.Cu) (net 29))
 (segment (start 172.97444 96.47599) (end 172.97444 79.12056) (width 0.25) (layer F.Cu) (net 27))
 (segment (start 172.97444 79.12056) (end 173.482 78.613) (width 0.25) (layer F.Cu) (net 27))
 (segment (start 173.482 78.613) (end 176.022 78.613) (width 0.25) (layer F.Cu) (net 27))
 (segment (start 176.022 78.613) (end 179.705 74.93) (width 0.25) (layer F.Cu) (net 27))
 (segment (start 179.705 74.93) (end 179.705 60.96) (width 0.25) (layer F.Cu) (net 27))
 (segment (start 142.113 113.284) (end 144.526 110.871) (width 0.25) (layer F.Cu) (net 27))
 (segment (start 172.847 97.663) (end 173.14945 97.663) (width 0.25) (layer F.Cu) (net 27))
 (segment (start 144.526 110.871) (end 159.639 110.871) (width 0.25) (layer F.Cu) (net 27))
 (segment (start 159.639 110.871) (end 172.847 97.663) (width 0.25) (layer F.Cu) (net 27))
 (segment (start 173.14945 97.663) (end 174.498 97.663) (width 0.25) (layer F.Cu) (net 27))
 (segment (start 174.498 97.663) (end 174.16145 97.663) (width 0.25) (layer F.Cu) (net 27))
 (segment (start 174.16145 97.663) (end 172.97444 96.47599) (width 0.25) (layer F.Cu) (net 27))
 (segment (start 172.974 96.47643) (end 172.97444 96.47599) (width 0.25) (layer F.Cu) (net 27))
 (segment (start 142.113 117.983) (end 142.113 113.284) (width 0.25) (layer B.Cu) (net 27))
 (via (at 142.113 113.284) (size 1.6) (drill 1) (layers F.Cu B.Cu) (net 27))
 (segment (start 143.24437 117.983) (end 142.113 117.983) (width 0.25) (layer F.Cu) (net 27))
 (segment (start 144.018 117.983) (end 143.24437 117.983) (width 0.25) (layer F.Cu) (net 27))
 (segment (start 145.288 117.983) (end 142.113 117.983) (width 0.25) (layer F.Cu) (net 27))
 (via (at 142.113 117.983) (size 1.6) (drill 1) (layers F.Cu B.Cu) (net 27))
 (segment (start 149.733 117.983) (end 145.288 117.983) (width 0.25) (layer F.Cu) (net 27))
 (segment (start 154.178 117.983) (end 149.733 117.983) (width 0.25) (layer F.Cu) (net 27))
 (segment (start 158.623 117.983) (end 154.178 117.983) (width 0.25) (layer F.Cu) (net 27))
 (segment (start 120.742135 81.474351) (end 120.742135 79.028865) (width 2.2) (layer F.Cu) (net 33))
 (segment (start 120.742135 79.028865) (end 124.968 74.803) (width 2.2) (layer F.Cu) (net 33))
 (segment (start 120.742135 89.094351) (end 120.742135 92.904351) (width 2.2) (layer F.Cu) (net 33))
 (segment (start 120.742135 85.284351) (end 120.742135 89.094351) (width 2.2) (layer F.Cu) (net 33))
 (segment (start 120.742135 81.474351) (end 120.742135 85.284351) (width 2.2) (layer F.Cu) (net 33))
 (segment (start 123.282135 92.904351) (end 123.282135 96.338965) (width 2.2) (layer F.Cu) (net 32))
 (segment (start 123.282135 96.338965) (end 120.015 99.6061) (width 2.2) (layer F.Cu) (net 32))
 (segment (start 123.317 92.939216) (end 123.282135 92.904351) (width 2.2) (layer F.Cu) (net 32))
 (segment (start 123.282135 89.094351) (end 123.282135 92.904351) (width 2.2) (layer F.Cu) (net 32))
 (segment (start 123.282135 85.284351) (end 123.282135 89.094351) (width 2.2) (layer F.Cu) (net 32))
 (segment (start 123.282135 81.474351) (end 123.282135 85.284351) (width 2.2) (layer F.Cu) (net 32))
 (segment (start 125.822135 89.094351) (end 125.822135 91.313) (width 2.2) (layer F.Cu) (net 31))
 (segment (start 125.822135 91.313) (end 125.822135 92.904351) (width 2.2) (layer F.Cu) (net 31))
 (segment (start 128.675784 95.758) (end 128.675784 94.166649) (width 2.2) (layer F.Cu) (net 31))
 (segment (start 128.675784 94.166649) (end 125.822135 91.313) (width 2.2) (layer F.Cu) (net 31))
 (segment (start 128.675784 104.545784) (end 133.223 109.093) (width 2.2) (layer F.Cu) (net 31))
 (segment (start 133.223 109.093) (end 133.223 109.2581) (width 2.2) (layer F.Cu) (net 31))
 (segment (start 128.675784 95.758) (end 128.675784 104.545784) (width 2.2) (layer F.Cu) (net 31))
 (segment (start 125.822135 85.284351) (end 125.822135 89.094351) (width 2.2) (layer F.Cu) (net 31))
 (segment (start 125.822135 81.474351) (end 125.822135 85.284351) (width 2.2) (layer F.Cu) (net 31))
 (segment (start 125.822135 92.904351) (end 125.822135 93.056751) (width 2.2) (layer F.Cu) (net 31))
 (segment (start 156.807001 113.575993) (end 157.607 112.775994) (width 0.25) (layer F.Cu) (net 30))
 (segment (start 155.574994 114.808) (end 156.807001 113.575993) (width 0.25) (layer F.Cu) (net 30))
 (segment (start 126.238 114.173) (end 126.873 114.808) (width 0.25) (layer F.Cu) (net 30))
 (segment (start 126.873 114.808) (end 155.574994 114.808) (width 0.25) (layer F.Cu) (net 30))
 (segment (start 126.238 108.458) (end 126.238 114.173) (width 0.25) (layer F.Cu) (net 30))
 (segment (start 124.333 106.553) (end 126.238 108.458) (width 0.25) (layer F.Cu) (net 30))
 (segment (start 112.903 95.123) (end 112.903 105.283) (width 0.25) (layer F.Cu) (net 30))
 (segment (start 114.173 106.553) (end 124.333 106.553) (width 0.25) (layer F.Cu) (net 30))
 (segment (start 112.903 105.283) (end 114.173 106.553) (width 0.25) (layer F.Cu) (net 30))
 (segment (start 115.121649 92.904351) (end 112.903 95.123) (width 0.25) (layer F.Cu) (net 30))
 (segment (start 118.202135 92.904351) (end 115.121649 92.904351) (width 0.25) (layer F.Cu) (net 30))
 (segment (start 164.592 112.776) (end 157.607006 112.776) (width 0.25) (layer B.Cu) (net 30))
 (segment (start 157.607006 112.776) (end 157.607 112.775994) (width 0.25) (layer B.Cu) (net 30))
 (via (at 157.607 112.775994) (size 1.6) (drill 1) (layers F.Cu B.Cu) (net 30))
 (segment (start 165.391999 111.976001) (end 164.592 112.776) (width 0.25) (layer F.Cu) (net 30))
 (segment (start 172.085 105.283) (end 165.391999 111.976001) (width 0.25) (layer F.Cu) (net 30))
 (segment (start 174.498 105.283) (end 172.085 105.283) (width 0.25) (layer F.Cu) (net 30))
 (via (at 164.592 112.776) (size 1.6) (drill 1) (layers F.Cu B.Cu) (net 30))
 (segment (start 113.538 84.963) (end 113.538 86.233) (width 2.2) (layer F.Cu) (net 30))
 (segment (start 113.538 83.693) (end 113.538 84.963) (width 2.2) (layer F.Cu) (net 30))
 (segment (start 113.538 84.963) (end 113.859351 85.284351) (width 2.2) (layer F.Cu) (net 30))
 (segment (start 113.859351 85.284351) (end 118.202135 85.284351) (width 2.2) (layer F.Cu) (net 30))
 (segment (start 118.202135 85.284351) (end 118.202135 87.503) (width 2.2) (layer F.Cu) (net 30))
 (segment (start 118.202135 87.503) (end 118.202135 89.094351) (width 2.2) (layer F.Cu) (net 30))
 (segment (start 118.202135 89.094351) (end 118.202135 92.904351) (width 2.2) (layer F.Cu) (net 30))
 (segment (start 118.202135 81.474351) (end 118.202135 85.284351) (width 2.2) (layer F.Cu) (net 30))
 (segment (start 172.593 76.78782) (end 172.593 64.258) (width 0.25) (layer F.Cu) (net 19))
 (segment (start 172.593 64.258) (end 174.625 62.226) (width 0.25) (layer F.Cu) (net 19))
 (segment (start 174.625 62.226) (end 174.625 60.96) (width 0.25) (layer F.Cu) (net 19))
 (segment (start 174.498 77.343) (end 173.14818 77.343) (width 0.25) (layer F.Cu) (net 19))
 (segment (start 173.14818 77.343) (end 172.593 76.78782) (width 0.25) (layer F.Cu) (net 19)))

